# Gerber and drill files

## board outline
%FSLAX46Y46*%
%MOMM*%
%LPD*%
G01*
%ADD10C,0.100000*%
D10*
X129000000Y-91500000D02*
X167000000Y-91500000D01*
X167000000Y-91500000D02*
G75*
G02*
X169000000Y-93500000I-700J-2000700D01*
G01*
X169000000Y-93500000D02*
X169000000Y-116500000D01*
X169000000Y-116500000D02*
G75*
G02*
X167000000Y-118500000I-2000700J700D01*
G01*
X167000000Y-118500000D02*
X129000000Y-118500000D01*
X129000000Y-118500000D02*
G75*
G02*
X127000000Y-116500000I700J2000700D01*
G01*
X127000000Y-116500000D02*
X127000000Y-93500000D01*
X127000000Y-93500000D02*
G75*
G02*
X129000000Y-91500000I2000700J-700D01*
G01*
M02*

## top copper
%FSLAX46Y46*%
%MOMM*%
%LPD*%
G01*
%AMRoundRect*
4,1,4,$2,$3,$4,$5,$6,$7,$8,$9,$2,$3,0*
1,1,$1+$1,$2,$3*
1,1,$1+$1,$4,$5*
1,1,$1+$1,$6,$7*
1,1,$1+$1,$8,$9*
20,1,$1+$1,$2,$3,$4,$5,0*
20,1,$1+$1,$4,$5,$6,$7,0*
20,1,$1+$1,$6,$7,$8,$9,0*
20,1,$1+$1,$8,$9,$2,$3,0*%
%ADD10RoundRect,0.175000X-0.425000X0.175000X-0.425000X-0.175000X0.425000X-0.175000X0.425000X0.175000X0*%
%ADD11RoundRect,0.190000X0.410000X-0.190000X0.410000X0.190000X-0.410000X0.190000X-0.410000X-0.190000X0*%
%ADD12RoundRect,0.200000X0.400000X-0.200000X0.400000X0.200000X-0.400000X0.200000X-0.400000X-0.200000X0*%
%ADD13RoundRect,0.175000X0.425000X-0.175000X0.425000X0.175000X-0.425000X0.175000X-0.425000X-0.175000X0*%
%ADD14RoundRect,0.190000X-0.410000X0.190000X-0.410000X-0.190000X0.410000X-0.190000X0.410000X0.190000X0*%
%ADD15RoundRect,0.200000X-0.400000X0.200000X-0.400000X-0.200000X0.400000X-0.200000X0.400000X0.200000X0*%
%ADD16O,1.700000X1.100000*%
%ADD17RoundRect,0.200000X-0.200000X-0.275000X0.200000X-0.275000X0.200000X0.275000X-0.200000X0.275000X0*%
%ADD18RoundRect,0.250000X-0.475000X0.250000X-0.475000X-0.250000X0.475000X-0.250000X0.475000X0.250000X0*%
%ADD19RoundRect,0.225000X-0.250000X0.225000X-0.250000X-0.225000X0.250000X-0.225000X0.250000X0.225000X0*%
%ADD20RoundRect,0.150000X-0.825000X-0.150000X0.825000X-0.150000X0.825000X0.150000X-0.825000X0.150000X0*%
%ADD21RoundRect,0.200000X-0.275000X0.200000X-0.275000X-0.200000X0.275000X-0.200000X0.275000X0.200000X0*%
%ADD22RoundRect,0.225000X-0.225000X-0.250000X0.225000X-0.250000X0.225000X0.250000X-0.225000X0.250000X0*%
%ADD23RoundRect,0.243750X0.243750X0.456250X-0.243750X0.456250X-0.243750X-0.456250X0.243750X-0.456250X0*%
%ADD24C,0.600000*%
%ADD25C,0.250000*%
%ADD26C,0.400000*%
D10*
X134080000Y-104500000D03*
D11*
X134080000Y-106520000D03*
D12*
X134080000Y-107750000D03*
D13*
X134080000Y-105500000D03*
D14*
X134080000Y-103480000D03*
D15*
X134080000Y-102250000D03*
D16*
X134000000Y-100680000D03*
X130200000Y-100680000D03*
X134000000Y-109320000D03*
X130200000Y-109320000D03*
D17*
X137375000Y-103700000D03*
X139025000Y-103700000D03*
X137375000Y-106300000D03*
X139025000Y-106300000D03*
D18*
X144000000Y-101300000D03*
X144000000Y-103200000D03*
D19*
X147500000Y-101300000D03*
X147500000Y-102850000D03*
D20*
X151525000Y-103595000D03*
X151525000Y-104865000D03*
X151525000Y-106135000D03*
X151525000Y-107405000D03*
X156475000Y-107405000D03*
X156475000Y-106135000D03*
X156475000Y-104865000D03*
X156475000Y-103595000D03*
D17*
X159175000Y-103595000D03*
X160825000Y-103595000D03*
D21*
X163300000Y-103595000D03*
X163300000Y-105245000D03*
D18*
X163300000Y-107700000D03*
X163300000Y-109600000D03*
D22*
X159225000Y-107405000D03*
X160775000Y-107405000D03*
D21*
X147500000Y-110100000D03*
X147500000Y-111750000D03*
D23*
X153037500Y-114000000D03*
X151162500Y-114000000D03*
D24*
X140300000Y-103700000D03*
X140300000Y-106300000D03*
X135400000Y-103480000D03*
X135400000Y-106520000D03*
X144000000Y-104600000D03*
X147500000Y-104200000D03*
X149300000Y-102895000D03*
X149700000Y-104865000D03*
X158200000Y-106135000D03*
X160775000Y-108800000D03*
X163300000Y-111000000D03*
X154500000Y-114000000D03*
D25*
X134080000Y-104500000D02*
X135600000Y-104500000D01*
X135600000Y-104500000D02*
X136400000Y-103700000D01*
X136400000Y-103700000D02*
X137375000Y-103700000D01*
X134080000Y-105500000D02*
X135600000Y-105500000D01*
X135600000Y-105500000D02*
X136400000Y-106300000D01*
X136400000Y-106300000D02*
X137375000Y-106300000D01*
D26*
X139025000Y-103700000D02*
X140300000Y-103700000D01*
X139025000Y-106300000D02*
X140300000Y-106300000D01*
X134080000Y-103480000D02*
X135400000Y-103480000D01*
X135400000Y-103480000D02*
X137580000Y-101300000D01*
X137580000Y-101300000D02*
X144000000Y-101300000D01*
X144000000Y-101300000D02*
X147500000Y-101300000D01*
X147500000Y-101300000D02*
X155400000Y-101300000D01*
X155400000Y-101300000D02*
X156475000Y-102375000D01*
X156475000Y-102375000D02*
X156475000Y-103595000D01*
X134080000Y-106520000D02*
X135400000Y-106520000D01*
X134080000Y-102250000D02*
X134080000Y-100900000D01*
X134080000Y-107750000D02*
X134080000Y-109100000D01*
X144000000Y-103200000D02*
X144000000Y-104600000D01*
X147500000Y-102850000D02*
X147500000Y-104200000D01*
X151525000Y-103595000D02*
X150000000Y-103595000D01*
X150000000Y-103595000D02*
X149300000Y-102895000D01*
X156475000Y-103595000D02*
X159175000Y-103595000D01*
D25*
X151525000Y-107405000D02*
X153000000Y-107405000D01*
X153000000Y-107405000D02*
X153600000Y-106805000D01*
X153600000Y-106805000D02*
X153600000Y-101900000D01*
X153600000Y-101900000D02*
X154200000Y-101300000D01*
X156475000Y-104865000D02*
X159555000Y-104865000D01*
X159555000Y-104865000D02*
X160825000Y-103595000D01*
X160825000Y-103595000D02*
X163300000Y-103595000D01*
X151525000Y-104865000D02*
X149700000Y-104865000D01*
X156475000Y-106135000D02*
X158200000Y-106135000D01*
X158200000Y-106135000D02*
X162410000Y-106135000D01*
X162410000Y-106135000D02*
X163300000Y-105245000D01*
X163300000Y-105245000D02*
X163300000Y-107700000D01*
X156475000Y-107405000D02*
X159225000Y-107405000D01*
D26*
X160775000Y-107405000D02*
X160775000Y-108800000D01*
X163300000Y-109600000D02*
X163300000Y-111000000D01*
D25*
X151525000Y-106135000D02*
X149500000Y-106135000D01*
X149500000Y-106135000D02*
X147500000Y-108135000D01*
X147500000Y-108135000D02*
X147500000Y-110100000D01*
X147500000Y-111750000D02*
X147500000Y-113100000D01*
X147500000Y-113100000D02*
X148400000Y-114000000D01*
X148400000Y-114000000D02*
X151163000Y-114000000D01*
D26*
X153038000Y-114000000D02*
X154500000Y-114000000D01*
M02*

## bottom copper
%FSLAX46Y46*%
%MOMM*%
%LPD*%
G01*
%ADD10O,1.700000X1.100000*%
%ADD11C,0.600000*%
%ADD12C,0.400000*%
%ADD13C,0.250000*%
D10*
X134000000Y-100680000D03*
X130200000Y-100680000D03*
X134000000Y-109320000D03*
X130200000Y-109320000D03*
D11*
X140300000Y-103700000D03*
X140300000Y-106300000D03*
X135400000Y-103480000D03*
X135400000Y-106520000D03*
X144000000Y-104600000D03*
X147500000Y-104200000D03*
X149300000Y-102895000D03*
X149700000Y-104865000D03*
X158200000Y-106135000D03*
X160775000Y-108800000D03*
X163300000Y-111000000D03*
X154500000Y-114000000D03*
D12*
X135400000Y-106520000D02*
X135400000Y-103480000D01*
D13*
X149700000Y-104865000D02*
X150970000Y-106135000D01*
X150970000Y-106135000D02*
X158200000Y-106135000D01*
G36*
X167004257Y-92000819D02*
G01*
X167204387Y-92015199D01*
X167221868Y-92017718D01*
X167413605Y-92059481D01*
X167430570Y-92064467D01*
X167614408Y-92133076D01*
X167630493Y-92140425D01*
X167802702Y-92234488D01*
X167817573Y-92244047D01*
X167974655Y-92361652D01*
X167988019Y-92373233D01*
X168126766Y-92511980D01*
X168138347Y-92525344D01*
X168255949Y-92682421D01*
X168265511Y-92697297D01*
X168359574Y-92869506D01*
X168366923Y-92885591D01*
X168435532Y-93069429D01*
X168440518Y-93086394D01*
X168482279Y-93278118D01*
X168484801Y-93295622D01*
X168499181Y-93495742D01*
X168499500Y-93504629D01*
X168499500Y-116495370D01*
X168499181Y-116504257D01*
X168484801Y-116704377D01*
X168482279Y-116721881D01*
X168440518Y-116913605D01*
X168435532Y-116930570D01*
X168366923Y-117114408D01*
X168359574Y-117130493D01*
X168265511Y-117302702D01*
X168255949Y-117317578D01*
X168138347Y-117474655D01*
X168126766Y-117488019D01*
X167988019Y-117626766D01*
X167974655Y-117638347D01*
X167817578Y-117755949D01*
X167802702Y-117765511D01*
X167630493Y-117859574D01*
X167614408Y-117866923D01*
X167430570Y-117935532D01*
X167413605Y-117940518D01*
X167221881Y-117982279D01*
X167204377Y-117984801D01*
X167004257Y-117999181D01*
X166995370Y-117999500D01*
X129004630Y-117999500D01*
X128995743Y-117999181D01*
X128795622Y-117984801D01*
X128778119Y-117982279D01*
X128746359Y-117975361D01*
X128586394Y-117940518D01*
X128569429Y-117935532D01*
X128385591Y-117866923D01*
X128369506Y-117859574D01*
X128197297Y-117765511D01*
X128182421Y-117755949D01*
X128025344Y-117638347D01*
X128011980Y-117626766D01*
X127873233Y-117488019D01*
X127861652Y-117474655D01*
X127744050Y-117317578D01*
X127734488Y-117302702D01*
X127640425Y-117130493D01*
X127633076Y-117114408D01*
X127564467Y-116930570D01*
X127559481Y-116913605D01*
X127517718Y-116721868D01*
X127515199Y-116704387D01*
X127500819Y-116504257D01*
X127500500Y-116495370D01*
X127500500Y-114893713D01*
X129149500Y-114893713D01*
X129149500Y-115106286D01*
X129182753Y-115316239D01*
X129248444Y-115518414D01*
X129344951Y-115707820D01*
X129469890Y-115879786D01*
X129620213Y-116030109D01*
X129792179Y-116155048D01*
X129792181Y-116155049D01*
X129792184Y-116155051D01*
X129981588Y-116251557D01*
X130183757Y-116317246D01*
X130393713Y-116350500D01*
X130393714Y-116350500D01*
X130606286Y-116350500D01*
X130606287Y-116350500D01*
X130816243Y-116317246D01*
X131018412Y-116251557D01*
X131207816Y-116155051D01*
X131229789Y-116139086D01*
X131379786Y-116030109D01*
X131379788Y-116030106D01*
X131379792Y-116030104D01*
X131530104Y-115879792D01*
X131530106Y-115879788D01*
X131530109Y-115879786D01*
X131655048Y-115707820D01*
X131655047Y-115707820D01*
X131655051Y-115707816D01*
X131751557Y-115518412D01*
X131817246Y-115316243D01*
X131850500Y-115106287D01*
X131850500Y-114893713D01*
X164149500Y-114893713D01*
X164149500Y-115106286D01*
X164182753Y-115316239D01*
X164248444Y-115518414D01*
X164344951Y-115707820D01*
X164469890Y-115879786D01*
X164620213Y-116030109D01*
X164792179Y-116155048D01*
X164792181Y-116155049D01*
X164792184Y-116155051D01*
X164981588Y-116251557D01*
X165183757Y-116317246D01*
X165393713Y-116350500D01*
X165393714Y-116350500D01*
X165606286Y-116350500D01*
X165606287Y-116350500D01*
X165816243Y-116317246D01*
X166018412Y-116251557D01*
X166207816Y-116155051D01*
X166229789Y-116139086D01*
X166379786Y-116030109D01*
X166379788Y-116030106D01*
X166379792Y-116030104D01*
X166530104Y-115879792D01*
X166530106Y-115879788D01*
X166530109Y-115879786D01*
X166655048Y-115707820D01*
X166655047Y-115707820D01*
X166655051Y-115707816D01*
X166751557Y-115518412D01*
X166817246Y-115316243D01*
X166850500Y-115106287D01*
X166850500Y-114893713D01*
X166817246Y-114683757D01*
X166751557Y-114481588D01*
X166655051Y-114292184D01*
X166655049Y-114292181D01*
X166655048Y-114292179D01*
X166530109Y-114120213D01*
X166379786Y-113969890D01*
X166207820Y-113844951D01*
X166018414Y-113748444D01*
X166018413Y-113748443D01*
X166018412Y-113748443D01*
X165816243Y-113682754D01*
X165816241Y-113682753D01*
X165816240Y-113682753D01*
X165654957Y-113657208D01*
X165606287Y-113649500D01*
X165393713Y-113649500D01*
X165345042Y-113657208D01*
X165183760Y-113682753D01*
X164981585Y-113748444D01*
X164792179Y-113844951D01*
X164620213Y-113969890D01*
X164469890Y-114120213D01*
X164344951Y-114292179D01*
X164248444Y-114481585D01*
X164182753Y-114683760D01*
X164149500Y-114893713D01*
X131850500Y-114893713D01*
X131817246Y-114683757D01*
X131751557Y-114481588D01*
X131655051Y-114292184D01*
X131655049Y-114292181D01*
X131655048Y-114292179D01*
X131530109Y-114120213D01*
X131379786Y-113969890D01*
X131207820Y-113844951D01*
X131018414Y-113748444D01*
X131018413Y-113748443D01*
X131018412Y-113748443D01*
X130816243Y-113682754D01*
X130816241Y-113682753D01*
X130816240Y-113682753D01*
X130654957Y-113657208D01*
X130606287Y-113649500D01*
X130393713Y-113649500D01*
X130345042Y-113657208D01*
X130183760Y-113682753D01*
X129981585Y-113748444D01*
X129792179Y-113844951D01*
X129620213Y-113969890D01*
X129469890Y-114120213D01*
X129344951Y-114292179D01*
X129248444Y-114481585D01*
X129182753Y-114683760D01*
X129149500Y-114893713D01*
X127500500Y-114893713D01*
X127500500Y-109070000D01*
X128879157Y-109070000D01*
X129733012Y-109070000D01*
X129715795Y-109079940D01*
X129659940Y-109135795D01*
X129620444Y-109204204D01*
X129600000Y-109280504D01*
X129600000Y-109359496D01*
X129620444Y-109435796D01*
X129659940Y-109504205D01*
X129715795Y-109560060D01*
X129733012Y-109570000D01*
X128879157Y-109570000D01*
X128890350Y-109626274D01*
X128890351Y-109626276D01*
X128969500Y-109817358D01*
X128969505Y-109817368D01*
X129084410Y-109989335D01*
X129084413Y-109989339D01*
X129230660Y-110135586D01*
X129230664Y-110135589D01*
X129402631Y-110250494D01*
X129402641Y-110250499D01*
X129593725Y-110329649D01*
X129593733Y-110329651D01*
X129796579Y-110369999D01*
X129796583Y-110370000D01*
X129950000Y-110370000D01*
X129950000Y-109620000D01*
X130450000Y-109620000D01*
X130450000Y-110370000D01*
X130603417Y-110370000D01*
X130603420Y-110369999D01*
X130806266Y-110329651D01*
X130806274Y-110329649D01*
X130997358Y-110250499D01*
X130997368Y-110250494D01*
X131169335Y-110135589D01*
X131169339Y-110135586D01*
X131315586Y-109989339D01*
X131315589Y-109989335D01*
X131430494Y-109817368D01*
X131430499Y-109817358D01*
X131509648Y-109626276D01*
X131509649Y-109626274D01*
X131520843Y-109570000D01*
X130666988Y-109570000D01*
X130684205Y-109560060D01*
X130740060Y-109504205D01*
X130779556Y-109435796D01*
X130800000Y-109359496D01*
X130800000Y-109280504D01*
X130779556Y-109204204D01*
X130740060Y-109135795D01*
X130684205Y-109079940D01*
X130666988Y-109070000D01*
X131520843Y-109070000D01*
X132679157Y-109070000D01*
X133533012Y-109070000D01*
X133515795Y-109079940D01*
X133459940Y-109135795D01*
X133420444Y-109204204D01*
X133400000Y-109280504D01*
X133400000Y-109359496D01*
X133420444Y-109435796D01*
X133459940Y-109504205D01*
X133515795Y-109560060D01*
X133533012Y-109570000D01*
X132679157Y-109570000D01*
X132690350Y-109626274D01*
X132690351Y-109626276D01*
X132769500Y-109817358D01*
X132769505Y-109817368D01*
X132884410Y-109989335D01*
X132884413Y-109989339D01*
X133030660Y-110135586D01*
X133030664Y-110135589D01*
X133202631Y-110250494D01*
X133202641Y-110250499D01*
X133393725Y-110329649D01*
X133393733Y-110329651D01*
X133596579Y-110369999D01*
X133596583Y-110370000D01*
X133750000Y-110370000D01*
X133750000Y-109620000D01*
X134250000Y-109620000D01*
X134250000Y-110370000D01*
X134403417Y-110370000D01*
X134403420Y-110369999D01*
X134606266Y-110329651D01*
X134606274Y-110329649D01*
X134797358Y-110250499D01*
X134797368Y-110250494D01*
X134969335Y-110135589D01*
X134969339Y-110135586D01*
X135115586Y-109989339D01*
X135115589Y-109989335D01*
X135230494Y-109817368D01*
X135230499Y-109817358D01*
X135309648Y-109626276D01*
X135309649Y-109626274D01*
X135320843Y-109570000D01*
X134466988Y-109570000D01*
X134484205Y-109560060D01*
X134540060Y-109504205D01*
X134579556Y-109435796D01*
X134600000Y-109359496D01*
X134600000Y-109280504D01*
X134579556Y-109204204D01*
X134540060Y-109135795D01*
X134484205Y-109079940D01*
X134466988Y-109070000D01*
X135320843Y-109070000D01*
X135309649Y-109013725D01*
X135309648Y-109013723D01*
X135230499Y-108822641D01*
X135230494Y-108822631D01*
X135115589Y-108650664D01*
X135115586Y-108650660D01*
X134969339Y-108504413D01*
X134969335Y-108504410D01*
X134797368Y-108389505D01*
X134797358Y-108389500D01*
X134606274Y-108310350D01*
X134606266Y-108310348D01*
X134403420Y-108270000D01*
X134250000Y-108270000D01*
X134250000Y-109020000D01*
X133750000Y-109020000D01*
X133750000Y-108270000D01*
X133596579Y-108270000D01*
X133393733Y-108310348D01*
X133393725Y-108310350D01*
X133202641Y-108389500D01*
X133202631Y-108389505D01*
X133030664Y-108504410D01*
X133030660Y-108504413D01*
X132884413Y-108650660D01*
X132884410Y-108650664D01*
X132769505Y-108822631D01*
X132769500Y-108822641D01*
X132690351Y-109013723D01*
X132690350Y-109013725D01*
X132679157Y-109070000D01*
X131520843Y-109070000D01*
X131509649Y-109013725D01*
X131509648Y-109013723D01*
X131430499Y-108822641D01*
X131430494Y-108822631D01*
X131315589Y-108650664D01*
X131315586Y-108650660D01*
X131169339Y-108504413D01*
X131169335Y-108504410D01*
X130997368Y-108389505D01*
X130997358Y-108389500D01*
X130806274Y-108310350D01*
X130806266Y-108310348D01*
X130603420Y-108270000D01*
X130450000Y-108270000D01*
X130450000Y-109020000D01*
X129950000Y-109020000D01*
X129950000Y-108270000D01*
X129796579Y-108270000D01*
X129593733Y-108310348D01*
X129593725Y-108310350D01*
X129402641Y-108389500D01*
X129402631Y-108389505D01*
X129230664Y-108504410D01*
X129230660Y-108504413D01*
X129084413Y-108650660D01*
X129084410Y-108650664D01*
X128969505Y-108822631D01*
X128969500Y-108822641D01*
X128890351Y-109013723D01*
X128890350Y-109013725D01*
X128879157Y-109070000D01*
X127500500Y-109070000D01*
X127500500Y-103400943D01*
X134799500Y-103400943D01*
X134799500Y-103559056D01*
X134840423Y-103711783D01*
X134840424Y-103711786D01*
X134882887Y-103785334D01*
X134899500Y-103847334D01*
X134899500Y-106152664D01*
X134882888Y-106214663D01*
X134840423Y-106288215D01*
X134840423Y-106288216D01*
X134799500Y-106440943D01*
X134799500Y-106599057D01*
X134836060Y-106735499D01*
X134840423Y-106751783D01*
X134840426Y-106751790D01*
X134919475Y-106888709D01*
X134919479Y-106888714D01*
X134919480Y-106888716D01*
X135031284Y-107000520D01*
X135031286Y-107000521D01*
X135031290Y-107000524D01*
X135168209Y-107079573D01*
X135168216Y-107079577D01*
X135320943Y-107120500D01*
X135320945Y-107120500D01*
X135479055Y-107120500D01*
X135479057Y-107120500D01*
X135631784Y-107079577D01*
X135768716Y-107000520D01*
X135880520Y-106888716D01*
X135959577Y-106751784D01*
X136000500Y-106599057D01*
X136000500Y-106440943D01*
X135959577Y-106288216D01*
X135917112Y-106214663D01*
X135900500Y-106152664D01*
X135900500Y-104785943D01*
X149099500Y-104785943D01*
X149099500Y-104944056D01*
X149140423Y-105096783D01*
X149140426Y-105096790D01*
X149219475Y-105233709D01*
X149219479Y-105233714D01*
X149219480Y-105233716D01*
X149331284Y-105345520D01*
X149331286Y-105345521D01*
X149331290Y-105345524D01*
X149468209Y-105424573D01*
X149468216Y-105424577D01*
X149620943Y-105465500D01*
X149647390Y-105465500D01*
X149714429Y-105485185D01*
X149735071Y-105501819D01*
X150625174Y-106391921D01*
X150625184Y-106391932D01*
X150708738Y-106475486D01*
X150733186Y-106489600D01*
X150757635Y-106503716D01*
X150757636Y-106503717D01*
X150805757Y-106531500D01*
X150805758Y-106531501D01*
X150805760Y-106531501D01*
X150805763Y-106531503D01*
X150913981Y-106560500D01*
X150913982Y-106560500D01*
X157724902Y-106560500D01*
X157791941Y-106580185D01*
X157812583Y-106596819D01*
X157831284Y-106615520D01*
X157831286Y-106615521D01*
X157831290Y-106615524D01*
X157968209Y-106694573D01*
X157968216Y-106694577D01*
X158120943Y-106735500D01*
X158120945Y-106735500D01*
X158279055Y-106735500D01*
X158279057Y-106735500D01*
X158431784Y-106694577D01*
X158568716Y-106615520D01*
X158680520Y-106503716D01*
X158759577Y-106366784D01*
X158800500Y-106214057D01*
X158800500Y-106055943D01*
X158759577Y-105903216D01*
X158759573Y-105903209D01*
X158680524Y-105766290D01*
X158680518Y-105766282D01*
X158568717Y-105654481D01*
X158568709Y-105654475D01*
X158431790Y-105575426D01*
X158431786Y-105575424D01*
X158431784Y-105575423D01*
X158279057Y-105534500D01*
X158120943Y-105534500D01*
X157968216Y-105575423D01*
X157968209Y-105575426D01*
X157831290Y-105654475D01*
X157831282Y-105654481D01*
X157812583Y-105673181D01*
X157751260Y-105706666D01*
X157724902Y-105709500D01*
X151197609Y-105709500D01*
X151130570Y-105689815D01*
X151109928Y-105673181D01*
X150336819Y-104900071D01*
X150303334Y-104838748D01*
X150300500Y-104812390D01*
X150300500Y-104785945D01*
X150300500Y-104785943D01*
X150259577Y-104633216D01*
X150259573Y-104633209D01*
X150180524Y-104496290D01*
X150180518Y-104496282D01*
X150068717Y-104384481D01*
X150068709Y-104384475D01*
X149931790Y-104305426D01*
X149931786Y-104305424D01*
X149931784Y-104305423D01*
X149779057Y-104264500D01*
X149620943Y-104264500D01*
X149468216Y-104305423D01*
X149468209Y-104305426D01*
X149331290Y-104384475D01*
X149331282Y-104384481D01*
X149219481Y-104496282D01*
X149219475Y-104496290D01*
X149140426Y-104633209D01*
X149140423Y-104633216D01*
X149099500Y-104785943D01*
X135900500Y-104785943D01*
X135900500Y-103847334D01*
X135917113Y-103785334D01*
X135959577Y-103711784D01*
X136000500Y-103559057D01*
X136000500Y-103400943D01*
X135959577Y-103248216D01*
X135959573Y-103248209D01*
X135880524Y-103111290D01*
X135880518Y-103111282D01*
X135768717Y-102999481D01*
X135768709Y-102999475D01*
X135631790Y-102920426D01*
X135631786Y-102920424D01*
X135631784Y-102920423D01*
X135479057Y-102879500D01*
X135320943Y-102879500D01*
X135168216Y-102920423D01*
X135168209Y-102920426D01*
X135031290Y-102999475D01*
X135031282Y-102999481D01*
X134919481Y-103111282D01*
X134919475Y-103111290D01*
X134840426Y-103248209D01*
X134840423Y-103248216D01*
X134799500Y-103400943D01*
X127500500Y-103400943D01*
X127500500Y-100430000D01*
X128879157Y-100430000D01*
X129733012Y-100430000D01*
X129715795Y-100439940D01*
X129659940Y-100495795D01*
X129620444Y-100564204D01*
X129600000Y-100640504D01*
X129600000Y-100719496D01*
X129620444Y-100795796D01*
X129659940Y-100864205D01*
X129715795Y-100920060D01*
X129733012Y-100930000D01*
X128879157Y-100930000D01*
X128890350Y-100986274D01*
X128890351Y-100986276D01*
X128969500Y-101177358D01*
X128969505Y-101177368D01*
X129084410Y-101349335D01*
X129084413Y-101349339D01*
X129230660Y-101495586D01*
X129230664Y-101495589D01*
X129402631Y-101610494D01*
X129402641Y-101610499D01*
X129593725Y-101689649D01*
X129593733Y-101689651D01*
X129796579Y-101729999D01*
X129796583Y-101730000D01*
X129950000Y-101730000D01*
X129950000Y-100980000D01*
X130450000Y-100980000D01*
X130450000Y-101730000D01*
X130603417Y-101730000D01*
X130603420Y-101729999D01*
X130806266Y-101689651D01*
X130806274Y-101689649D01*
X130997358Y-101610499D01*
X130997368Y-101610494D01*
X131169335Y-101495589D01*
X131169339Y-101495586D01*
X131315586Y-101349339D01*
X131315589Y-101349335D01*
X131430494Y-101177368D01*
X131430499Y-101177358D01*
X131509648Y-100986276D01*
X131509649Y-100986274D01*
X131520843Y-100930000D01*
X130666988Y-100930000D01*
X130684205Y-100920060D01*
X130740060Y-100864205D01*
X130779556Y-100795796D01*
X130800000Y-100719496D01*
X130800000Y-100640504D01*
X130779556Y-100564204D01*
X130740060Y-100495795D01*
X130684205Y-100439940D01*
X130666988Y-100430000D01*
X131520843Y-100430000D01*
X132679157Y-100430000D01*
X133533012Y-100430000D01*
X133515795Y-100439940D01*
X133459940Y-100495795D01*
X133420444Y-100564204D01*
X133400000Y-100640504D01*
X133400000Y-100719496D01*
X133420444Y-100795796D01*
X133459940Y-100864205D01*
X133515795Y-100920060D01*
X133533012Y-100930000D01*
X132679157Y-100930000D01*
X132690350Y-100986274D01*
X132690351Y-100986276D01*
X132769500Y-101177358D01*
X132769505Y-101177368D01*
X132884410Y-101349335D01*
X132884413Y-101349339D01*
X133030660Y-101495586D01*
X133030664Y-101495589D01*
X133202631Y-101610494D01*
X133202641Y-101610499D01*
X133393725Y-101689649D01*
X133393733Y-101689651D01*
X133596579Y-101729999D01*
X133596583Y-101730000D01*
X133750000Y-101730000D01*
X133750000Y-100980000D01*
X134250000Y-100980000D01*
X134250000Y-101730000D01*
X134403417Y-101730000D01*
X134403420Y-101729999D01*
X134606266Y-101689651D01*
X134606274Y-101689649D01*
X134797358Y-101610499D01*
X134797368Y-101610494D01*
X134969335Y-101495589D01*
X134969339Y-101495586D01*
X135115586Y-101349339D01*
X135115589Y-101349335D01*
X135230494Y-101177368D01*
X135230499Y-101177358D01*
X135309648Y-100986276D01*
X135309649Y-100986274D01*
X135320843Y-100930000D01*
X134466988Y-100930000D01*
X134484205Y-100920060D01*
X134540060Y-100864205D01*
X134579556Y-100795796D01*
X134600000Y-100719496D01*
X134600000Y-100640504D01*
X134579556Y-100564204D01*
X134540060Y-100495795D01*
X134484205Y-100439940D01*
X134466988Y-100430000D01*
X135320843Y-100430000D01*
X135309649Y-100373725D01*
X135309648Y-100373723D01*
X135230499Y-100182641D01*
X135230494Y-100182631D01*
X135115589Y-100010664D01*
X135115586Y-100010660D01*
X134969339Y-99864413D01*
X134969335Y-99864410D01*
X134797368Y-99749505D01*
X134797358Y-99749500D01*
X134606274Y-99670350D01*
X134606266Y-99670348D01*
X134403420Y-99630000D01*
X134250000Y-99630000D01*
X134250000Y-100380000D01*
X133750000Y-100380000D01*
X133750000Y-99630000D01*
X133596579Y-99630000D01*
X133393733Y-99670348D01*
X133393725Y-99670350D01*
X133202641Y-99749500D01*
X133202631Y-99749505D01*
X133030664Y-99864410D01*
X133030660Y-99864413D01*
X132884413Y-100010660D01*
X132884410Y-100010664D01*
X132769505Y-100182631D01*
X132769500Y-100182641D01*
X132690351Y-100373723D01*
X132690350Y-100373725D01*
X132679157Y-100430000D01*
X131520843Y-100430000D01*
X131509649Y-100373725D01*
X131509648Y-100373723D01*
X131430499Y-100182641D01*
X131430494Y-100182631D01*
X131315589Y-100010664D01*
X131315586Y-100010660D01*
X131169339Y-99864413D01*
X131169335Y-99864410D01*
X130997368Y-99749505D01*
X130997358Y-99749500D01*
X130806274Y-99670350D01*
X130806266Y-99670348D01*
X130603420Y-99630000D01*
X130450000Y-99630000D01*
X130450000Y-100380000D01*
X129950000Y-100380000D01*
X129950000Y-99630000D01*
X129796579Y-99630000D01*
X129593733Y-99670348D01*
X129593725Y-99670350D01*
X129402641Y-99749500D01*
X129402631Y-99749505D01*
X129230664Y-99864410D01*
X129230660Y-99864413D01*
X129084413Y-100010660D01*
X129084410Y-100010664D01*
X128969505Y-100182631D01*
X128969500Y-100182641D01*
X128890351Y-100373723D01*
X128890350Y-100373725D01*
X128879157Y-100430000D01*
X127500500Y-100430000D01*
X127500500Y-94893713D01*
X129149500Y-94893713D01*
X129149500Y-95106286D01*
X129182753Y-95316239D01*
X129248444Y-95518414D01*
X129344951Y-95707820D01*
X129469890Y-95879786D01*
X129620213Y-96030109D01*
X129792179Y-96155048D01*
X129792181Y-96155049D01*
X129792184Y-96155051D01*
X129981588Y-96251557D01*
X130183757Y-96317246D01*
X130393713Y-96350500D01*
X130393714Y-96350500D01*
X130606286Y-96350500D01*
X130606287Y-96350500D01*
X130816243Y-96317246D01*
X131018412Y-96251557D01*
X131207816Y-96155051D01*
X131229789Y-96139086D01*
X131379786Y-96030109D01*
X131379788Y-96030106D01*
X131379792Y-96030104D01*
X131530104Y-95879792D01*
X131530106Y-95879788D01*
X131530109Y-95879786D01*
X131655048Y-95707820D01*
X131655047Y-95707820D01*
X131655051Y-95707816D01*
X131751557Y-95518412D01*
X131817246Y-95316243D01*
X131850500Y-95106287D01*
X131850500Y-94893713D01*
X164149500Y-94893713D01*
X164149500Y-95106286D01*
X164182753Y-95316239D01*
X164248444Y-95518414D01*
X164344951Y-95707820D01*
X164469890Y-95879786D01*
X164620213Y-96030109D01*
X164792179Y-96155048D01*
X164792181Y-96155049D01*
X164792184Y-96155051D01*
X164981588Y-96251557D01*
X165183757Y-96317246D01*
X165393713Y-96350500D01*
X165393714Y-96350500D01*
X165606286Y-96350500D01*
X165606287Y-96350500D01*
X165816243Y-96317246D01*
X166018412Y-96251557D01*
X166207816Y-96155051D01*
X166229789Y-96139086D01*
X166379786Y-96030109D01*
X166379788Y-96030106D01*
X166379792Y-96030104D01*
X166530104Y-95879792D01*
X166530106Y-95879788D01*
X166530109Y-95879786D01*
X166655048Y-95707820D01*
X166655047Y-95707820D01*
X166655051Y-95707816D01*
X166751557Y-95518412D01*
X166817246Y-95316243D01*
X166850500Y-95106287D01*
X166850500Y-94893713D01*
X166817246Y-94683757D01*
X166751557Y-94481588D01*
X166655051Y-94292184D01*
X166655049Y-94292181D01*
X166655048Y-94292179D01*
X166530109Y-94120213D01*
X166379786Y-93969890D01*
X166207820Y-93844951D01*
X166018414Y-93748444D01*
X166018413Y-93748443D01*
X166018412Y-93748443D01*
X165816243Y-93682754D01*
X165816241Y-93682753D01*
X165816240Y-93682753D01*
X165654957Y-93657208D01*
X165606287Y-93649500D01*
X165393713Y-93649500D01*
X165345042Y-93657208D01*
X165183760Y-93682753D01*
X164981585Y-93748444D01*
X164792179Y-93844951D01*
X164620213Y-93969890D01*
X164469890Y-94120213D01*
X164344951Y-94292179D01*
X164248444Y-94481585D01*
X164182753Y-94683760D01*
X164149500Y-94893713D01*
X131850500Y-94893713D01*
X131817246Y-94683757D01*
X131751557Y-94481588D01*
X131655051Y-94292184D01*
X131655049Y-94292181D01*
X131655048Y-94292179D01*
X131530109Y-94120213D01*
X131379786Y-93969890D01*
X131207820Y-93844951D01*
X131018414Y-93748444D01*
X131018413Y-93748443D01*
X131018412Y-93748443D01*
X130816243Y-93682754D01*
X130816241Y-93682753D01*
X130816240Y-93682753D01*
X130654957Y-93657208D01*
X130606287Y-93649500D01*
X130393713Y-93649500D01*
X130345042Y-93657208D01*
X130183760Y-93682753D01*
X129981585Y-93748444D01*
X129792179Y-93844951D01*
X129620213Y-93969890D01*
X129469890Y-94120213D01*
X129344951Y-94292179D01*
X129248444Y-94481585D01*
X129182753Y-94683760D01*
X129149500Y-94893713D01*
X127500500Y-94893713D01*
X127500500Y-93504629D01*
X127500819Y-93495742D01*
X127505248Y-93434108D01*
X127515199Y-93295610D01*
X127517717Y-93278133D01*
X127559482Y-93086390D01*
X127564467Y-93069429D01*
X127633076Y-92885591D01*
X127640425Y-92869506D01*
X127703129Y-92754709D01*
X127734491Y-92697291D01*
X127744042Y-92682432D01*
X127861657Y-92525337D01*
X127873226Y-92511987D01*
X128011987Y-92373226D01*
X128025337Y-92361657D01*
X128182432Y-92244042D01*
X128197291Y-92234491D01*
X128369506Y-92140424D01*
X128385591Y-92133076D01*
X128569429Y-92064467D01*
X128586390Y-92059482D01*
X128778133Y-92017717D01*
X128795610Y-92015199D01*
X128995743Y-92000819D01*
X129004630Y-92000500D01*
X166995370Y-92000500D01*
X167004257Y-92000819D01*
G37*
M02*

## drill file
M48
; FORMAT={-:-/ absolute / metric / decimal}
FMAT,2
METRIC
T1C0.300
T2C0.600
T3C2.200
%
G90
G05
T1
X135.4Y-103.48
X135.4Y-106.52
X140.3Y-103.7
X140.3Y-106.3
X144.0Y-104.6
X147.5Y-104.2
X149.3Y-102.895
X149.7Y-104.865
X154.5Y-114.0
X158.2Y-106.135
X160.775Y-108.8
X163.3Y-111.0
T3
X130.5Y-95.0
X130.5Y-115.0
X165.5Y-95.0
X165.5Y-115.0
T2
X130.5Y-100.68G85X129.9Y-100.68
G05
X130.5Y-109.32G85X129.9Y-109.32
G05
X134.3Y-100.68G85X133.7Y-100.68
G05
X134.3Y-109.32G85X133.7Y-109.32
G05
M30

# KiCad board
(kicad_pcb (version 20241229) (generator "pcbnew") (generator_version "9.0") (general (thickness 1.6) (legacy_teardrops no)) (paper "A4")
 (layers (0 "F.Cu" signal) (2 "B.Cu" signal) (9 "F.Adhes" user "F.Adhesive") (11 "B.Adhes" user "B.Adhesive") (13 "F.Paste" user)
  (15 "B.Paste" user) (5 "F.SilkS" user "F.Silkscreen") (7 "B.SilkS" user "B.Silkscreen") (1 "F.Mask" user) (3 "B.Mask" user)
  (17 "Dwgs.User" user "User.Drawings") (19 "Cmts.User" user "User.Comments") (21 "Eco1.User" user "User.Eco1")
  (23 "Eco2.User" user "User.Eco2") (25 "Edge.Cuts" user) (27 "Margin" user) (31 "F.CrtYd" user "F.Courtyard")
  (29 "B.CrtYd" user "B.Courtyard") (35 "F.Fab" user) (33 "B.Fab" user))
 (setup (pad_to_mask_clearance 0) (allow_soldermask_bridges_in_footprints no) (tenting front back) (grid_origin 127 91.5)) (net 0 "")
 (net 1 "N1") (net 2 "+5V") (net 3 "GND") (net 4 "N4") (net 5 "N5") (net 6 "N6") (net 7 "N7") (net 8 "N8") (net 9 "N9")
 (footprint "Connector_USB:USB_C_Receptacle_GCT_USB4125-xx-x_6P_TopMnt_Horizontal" (layer "F.Cu") (at 131 105 270)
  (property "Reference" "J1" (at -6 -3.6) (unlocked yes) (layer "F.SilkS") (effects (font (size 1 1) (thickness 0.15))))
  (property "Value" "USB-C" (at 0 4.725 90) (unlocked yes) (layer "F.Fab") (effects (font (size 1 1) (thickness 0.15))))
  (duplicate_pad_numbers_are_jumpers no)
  (pad "A5" smd roundrect (at -0.5 -3.08 270) (size 0.7 1.2) (layers "F.Cu" "F.Mask" "F.Paste") (roundrect_rratio 0.25) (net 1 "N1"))
  (pad "A9" smd roundrect (at 1.52 -3.08 90) (size 0.76 1.2) (layers "F.Cu" "F.Mask" "F.Paste") (roundrect_rratio 0.25) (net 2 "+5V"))
  (pad "A12" smd roundrect (at 2.75 -3.08 90) (size 0.8 1.2) (layers "F.Cu" "F.Mask" "F.Paste") (roundrect_rratio 0.25) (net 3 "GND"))
  (pad "B5" smd roundrect (at 0.5 -3.08 90) (size 0.7 1.2) (layers "F.Cu" "F.Mask" "F.Paste") (roundrect_rratio 0.25) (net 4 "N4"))
  (pad "B9" smd roundrect (at -1.52 -3.08 270) (size 0.76 1.2) (layers "F.Cu" "F.Mask" "F.Paste") (roundrect_rratio 0.25) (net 2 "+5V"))
  (pad "B12" smd roundrect (at -2.75 -3.08 270) (size 0.8 1.2) (layers "F.Cu" "F.Mask" "F.Paste") (roundrect_rratio 0.25) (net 3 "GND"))
  (pad "SH" thru_hole oval (at -4.32 -3 270) (size 1.1 1.7) (drill oval 0.6 1.2) (layers "*.Cu" "*.Mask" "F.Paste")
   (remove_unused_layers no) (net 3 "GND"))
  (pad "SH" thru_hole oval (at -4.32 0.8 270) (size 1.1 1.7) (drill oval 0.6 1.2) (layers "*.Cu" "*.Mask" "F.Paste")
   (remove_unused_layers no) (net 3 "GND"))
  (pad "SH" thru_hole oval (at 4.32 -3 270) (size 1.1 1.7) (drill oval 0.6 1.2) (layers "*.Cu" "*.Mask" "F.Paste") (remove_unused_layers no)
   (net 3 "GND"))
  (pad "SH" thru_hole oval (at 4.32 0.8 270) (size 1.1 1.7) (drill oval 0.6 1.2) (layers "*.Cu" "*.Mask" "F.Paste")
   (remove_unused_layers no) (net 3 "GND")))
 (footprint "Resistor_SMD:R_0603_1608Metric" (layer "F.Cu") (at 138.2 103.7)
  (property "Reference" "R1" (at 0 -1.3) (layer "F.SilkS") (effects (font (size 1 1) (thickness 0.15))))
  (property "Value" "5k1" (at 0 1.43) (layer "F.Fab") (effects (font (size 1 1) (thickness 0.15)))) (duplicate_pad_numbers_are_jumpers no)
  (pad "1" smd roundrect (at -0.825 0) (size 0.8 0.95) (layers "F.Cu" "F.Mask" "F.Paste") (roundrect_rratio 0.25) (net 1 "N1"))
  (pad "2" smd roundrect (at 0.825 0) (size 0.8 0.95) (layers "F.Cu" "F.Mask" "F.Paste") (roundrect_rratio 0.25) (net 3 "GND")))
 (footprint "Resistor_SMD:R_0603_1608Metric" (layer "F.Cu") (at 138.2 106.3)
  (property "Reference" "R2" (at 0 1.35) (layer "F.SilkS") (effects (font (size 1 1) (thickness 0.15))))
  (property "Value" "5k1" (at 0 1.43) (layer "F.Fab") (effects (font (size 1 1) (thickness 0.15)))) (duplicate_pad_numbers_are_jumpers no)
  (pad "1" smd roundrect (at -0.825 0) (size 0.8 0.95) (layers "F.Cu" "F.Mask" "F.Paste") (roundrect_rratio 0.25) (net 4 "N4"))
  (pad "2" smd roundrect (at 0.825 0) (size 0.8 0.95) (layers "F.Cu" "F.Mask" "F.Paste") (roundrect_rratio 0.25) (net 3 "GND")))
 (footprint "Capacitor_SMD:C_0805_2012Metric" (layer "F.Cu") (at 144 102.25 270)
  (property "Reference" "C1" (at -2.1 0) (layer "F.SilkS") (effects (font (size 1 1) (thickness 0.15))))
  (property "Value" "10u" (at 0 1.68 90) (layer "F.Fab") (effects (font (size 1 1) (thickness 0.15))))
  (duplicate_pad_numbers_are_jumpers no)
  (pad "1" smd roundrect (at -0.95 0 270) (size 1 1.45) (layers "F.Cu" "F.Mask" "F.Paste") (roundrect_rratio 0.25) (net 2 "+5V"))
  (pad "2" smd roundrect (at 0.95 0 270) (size 1 1.45) (layers "F.Cu" "F.Mask" "F.Paste") (roundrect_rratio 0.25) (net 3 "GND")))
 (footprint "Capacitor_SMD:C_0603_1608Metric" (layer "F.Cu") (at 147.5 102.075 270)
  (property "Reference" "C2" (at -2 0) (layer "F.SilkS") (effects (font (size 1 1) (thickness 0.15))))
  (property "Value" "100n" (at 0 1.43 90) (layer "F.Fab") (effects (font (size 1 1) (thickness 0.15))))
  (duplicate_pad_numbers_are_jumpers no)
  (pad "1" smd roundrect (at -0.775 0 270) (size 0.9 0.95) (layers "F.Cu" "F.Mask" "F.Paste") (roundrect_rratio 0.25) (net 2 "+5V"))
  (pad "2" smd roundrect (at 0.775 0 270) (size 0.9 0.95) (layers "F.Cu" "F.Mask" "F.Paste") (roundrect_rratio 0.25) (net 3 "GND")))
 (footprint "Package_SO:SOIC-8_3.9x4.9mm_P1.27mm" (layer "F.Cu") (at 154 105.5)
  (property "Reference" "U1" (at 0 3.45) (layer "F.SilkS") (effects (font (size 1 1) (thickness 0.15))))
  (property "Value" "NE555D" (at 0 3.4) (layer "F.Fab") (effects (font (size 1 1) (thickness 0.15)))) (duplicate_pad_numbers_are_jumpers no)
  (pad "1" smd roundrect (at -2.475 -1.905) (size 1.95 0.6) (layers "F.Cu" "F.Mask" "F.Paste") (roundrect_rratio 0.25) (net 3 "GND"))
  (pad "2" smd roundrect (at -2.475 -0.635) (size 1.95 0.6) (layers "F.Cu" "F.Mask" "F.Paste") (roundrect_rratio 0.25) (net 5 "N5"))
  (pad "3" smd roundrect (at -2.475 0.635) (size 1.95 0.6) (layers "F.Cu" "F.Mask" "F.Paste") (roundrect_rratio 0.25) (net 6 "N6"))
  (pad "4" smd roundrect (at -2.475 1.905) (size 1.95 0.6) (layers "F.Cu" "F.Mask" "F.Paste") (roundrect_rratio 0.25) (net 2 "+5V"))
  (pad "5" smd roundrect (at 2.475 1.905) (size 1.95 0.6) (layers "F.Cu" "F.Mask" "F.Paste") (roundrect_rratio 0.25) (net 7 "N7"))
  (pad "6" smd roundrect (at 2.475 0.635) (size 1.95 0.6) (layers "F.Cu" "F.Mask" "F.Paste") (roundrect_rratio 0.25) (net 5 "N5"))
  (pad "7" smd roundrect (at 2.475 -0.635) (size 1.95 0.6) (layers "F.Cu" "F.Mask" "F.Paste") (roundrect_rratio 0.25) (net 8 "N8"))
  (pad "8" smd roundrect (at 2.475 -1.905) (size 1.95 0.6) (layers "F.Cu" "F.Mask" "F.Paste") (roundrect_rratio 0.25) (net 2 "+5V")))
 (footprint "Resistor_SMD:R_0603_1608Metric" (layer "F.Cu") (at 160 103.595)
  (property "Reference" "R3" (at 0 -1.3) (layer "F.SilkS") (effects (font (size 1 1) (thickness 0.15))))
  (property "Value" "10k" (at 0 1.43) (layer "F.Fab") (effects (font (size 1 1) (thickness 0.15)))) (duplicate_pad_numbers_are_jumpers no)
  (pad "1" smd roundrect (at -0.825 0) (size 0.8 0.95) (layers "F.Cu" "F.Mask" "F.Paste") (roundrect_rratio 0.25) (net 2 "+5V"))
  (pad "2" smd roundrect (at 0.825 0) (size 0.8 0.95) (layers "F.Cu" "F.Mask" "F.Paste") (roundrect_rratio 0.25) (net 8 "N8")))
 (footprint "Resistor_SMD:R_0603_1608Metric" (layer "F.Cu") (at 163.3 104.42 270)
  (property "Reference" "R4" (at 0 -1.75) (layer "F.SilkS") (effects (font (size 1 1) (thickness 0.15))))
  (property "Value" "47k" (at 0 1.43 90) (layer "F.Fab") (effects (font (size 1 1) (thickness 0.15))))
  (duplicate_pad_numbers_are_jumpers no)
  (pad "1" smd roundrect (at -0.825 0 270) (size 0.8 0.95) (layers "F.Cu" "F.Mask" "F.Paste") (roundrect_rratio 0.25) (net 8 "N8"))
  (pad "2" smd roundrect (at 0.825 0 270) (size 0.8 0.95) (layers "F.Cu" "F.Mask" "F.Paste") (roundrect_rratio 0.25) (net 5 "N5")))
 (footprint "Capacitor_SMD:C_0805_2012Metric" (layer "F.Cu") (at 163.3 108.65 270)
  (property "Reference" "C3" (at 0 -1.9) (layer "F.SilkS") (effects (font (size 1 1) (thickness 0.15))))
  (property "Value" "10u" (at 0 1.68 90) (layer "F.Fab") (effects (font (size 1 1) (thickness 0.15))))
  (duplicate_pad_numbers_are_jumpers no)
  (pad "1" smd roundrect (at -0.95 0 270) (size 1 1.45) (layers "F.Cu" "F.Mask" "F.Paste") (roundrect_rratio 0.25) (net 5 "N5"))
  (pad "2" smd roundrect (at 0.95 0 270) (size 1 1.45) (layers "F.Cu" "F.Mask" "F.Paste") (roundrect_rratio 0.25) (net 3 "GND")))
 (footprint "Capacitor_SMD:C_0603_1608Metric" (layer "F.Cu") (at 160 107.405)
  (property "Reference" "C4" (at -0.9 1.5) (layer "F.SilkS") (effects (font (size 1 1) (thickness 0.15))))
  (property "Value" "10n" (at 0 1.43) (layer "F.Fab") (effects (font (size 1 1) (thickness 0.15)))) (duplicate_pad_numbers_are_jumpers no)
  (pad "1" smd roundrect (at -0.775 0) (size 0.9 0.95) (layers "F.Cu" "F.Mask" "F.Paste") (roundrect_rratio 0.25) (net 7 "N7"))
  (pad "2" smd roundrect (at 0.775 0) (size 0.9 0.95) (layers "F.Cu" "F.Mask" "F.Paste") (roundrect_rratio 0.25) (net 3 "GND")))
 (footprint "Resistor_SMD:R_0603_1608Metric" (layer "F.Cu") (at 147.5 110.925 270)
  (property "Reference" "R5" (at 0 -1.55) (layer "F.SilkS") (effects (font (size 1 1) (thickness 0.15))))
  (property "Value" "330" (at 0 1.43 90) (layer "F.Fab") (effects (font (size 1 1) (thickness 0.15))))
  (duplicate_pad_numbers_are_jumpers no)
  (pad "1" smd roundrect (at -0.825 0 270) (size 0.8 0.95) (layers "F.Cu" "F.Mask" "F.Paste") (roundrect_rratio 0.25) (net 6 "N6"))
  (pad "2" smd roundrect (at 0.825 0 270) (size 0.8 0.95) (layers "F.Cu" "F.Mask" "F.Paste") (roundrect_rratio 0.25) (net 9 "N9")))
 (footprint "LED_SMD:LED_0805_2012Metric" (layer "F.Cu") (at 152.1 114 180)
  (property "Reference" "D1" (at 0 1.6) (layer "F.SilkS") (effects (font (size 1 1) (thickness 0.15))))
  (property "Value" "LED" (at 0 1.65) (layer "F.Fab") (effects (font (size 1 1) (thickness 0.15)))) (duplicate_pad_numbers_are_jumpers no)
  (pad "1" smd roundrect (at -0.9375 0 180) (size 0.975 1.4) (layers "F.Cu" "F.Mask" "F.Paste") (roundrect_rratio 0.25) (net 3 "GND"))
  (pad "2" smd roundrect (at 0.9375 0 180) (size 0.975 1.4) (layers "F.Cu" "F.Mask" "F.Paste") (roundrect_rratio 0.25) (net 9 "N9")))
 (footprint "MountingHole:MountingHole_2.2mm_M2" (layer "F.Cu") (at 130.5 95)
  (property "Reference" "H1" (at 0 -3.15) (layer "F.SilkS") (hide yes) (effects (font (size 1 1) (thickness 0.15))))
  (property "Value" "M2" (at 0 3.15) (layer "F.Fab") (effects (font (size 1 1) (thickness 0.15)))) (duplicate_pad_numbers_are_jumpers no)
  (pad "" np_thru_hole circle (at 0 0) (size 2.2 2.2) (drill 2.2) (layers "*.Cu" "*.Mask")))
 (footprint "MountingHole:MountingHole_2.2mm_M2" (layer "F.Cu") (at 165.5 95)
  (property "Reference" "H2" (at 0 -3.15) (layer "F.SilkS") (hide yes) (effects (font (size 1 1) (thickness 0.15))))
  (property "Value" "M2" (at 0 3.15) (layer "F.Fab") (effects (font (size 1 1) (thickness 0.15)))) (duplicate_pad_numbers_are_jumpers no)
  (pad "" np_thru_hole circle (at 0 0) (size 2.2 2.2) (drill 2.2) (layers "*.Cu" "*.Mask")))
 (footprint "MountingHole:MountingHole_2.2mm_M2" (layer "F.Cu") (at 130.5 115)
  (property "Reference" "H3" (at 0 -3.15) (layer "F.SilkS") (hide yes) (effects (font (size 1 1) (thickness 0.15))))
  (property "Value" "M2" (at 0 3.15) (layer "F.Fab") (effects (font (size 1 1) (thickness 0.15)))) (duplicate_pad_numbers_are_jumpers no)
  (pad "" np_thru_hole circle (at 0 0) (size 2.2 2.2) (drill 2.2) (layers "*.Cu" "*.Mask")))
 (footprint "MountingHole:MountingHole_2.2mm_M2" (layer "F.Cu") (at 165.5 115)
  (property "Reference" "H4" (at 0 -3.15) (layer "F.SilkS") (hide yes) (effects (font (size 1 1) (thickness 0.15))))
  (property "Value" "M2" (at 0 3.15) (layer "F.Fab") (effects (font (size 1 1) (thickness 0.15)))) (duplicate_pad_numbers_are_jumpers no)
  (pad "" np_thru_hole circle (at 0 0) (size 2.2 2.2) (drill 2.2) (layers "*.Cu" "*.Mask")))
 (segment (start 134.08 104.5) (end 135.6 104.5) (width 0.25) (layer "F.Cu") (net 1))
 (segment (start 135.6 104.5) (end 136.4 103.7) (width 0.25) (layer "F.Cu") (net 1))
 (segment (start 136.4 103.7) (end 137.375 103.7) (width 0.25) (layer "F.Cu") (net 1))
 (segment (start 134.08 105.5) (end 135.6 105.5) (width 0.25) (layer "F.Cu") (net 4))
 (segment (start 135.6 105.5) (end 136.4 106.3) (width 0.25) (layer "F.Cu") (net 4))
 (segment (start 136.4 106.3) (end 137.375 106.3) (width 0.25) (layer "F.Cu") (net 4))
 (segment (start 139.025 103.7) (end 140.3 103.7) (width 0.4) (layer "F.Cu") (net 3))
 (via (at 140.3 103.7) (size 0.6) (drill 0.3) (layers "F.Cu" "B.Cu") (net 3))
 (segment (start 139.025 106.3) (end 140.3 106.3) (width 0.4) (layer "F.Cu") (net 3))
 (via (at 140.3 106.3) (size 0.6) (drill 0.3) (layers "F.Cu" "B.Cu") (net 3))
 (segment (start 134.08 103.48) (end 135.4 103.48) (width 0.4) (layer "F.Cu") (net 2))
 (via (at 135.4 103.48) (size 0.6) (drill 0.3) (layers "F.Cu" "B.Cu") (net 2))
 (segment (start 135.4 103.48) (end 137.58 101.3) (width 0.4) (layer "F.Cu") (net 2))
 (segment (start 137.58 101.3) (end 144 101.3) (width 0.4) (layer "F.Cu") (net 2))
 (segment (start 144 101.3) (end 147.5 101.3) (width 0.4) (layer "F.Cu") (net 2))
 (segment (start 147.5 101.3) (end 155.4 101.3) (width 0.4) (layer "F.Cu") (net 2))
 (segment (start 155.4 101.3) (end 156.475 102.375) (width 0.4) (layer "F.Cu") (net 2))
 (segment (start 156.475 102.375) (end 156.475 103.595) (width 0.4) (layer "F.Cu") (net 2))
 (segment (start 134.08 106.52) (end 135.4 106.52) (width 0.4) (layer "F.Cu") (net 2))
 (via (at 135.4 106.52) (size 0.6) (drill 0.3) (layers "F.Cu" "B.Cu") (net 2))
 (segment (start 135.4 106.52) (end 135.4 103.48) (width 0.4) (layer "B.Cu") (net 2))
 (segment (start 134.08 102.25) (end 134.08 100.9) (width 0.4) (layer "F.Cu") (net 3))
 (segment (start 134.08 107.75) (end 134.08 109.1) (width 0.4) (layer "F.Cu") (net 3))
 (segment (start 144 103.2) (end 144 104.6) (width 0.4) (layer "F.Cu") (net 3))
 (via (at 144 104.6) (size 0.6) (drill 0.3) (layers "F.Cu" "B.Cu") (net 3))
 (segment (start 147.5 102.85) (end 147.5 104.2) (width 0.4) (layer "F.Cu") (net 3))
 (via (at 147.5 104.2) (size 0.6) (drill 0.3) (layers "F.Cu" "B.Cu") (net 3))
 (segment (start 151.525 103.595) (end 150 103.595) (width 0.4) (layer "F.Cu") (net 3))
 (segment (start 150 103.595) (end 149.3 102.895) (width 0.4) (layer "F.Cu") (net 3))
 (via (at 149.3 102.895) (size 0.6) (drill 0.3) (layers "F.Cu" "B.Cu") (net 3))
 (segment (start 156.475 103.595) (end 159.175 103.595) (width 0.4) (layer "F.Cu") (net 2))
 (segment (start 151.525 107.405) (end 153 107.405) (width 0.25) (layer "F.Cu") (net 2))
 (segment (start 153 107.405) (end 153.6 106.805) (width 0.25) (layer "F.Cu") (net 2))
 (segment (start 153.6 106.805) (end 153.6 101.9) (width 0.25) (layer "F.Cu") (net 2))
 (segment (start 153.6 101.9) (end 154.2 101.3) (width 0.25) (layer "F.Cu") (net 2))
 (segment (start 156.475 104.865) (end 159.555 104.865) (width 0.25) (layer "F.Cu") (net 8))
 (segment (start 159.555 104.865) (end 160.825 103.595) (width 0.25) (layer "F.Cu") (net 8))
 (segment (start 160.825 103.595) (end 163.3 103.595) (width 0.25) (layer "F.Cu") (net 8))
 (segment (start 151.525 104.865) (end 149.7 104.865) (width 0.25) (layer "F.Cu") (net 5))
 (via (at 149.7 104.865) (size 0.6) (drill 0.3) (layers "F.Cu" "B.Cu") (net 5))
 (segment (start 149.7 104.865) (end 150.97 106.135) (width 0.25) (layer "B.Cu") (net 5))
 (segment (start 150.97 106.135) (end 158.2 106.135) (width 0.25) (layer "B.Cu") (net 5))
 (via (at 158.2 106.135) (size 0.6) (drill 0.3) (layers "F.Cu" "B.Cu") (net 5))
 (segment (start 156.475 106.135) (end 158.2 106.135) (width 0.25) (layer "F.Cu") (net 5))
 (segment (start 158.2 106.135) (end 162.41 106.135) (width 0.25) (layer "F.Cu") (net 5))
 (segment (start 162.41 106.135) (end 163.3 105.245) (width 0.25) (layer "F.Cu") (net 5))
 (segment (start 163.3 105.245) (end 163.3 107.7) (width 0.25) (layer "F.Cu") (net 5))
 (segment (start 156.475 107.405) (end 159.225 107.405) (width 0.25) (layer "F.Cu") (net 7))
 (segment (start 160.775 107.405) (end 160.775 108.8) (width 0.4) (layer "F.Cu") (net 3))
 (via (at 160.775 108.8) (size 0.6) (drill 0.3) (layers "F.Cu" "B.Cu") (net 3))
 (segment (start 163.3 109.6) (end 163.3 111) (width 0.4) (layer "F.Cu") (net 3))
 (via (at 163.3 111) (size 0.6) (drill 0.3) (layers "F.Cu" "B.Cu") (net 3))
 (segment (start 151.525 106.135) (end 149.5 106.135) (width 0.25) (layer "F.Cu") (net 6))
 (segment (start 149.5 106.135) (end 147.5 108.135) (width 0.25) (layer "F.Cu") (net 6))
 (segment (start 147.5 108.135) (end 147.5 110.1) (width 0.25) (layer "F.Cu") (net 6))
 (segment (start 147.5 111.75) (end 147.5 113.1) (width 0.25) (layer "F.Cu") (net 9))
 (segment (start 147.5 113.1) (end 148.4 114) (width 0.25) (layer "F.Cu") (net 9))
 (segment (start 148.4 114) (end 151.163 114) (width 0.25) (layer "F.Cu") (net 9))
 (segment (start 153.038 114) (end 154.5 114) (width 0.4) (layer "F.Cu") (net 3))
 (via (at 154.5 114) (size 0.6) (drill 0.3) (layers "F.Cu" "B.Cu") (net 3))
 (gr_line (start 129 91.5) (end 167 91.5) (stroke (width 0.1) (type default)) (layer "Edge.Cuts"))
 (gr_arc (start 167 91.5) (mid 168.414 92.086) (end 169 93.5) (stroke (width 0.1) (type default)) (layer "Edge.Cuts"))
 (gr_line (start 169 93.5) (end 169 116.5) (stroke (width 0.1) (type default)) (layer "Edge.Cuts"))
 (gr_arc (start 169 116.5) (mid 168.414 117.914) (end 167 118.5) (stroke (width 0.1) (type default)) (layer "Edge.Cuts"))
 (gr_line (start 167 118.5) (end 129 118.5) (stroke (width 0.1) (type default)) (layer "Edge.Cuts"))
 (gr_arc (start 129 118.5) (mid 127.586 117.914) (end 127 116.5) (stroke (width 0.1) (type default)) (layer "Edge.Cuts"))
 (gr_line (start 127 116.5) (end 127 93.5) (stroke (width 0.1) (type default)) (layer "Edge.Cuts"))
 (gr_arc (start 127 93.5) (mid 127.586 92.086) (end 129 91.5) (stroke (width 0.1) (type default)) (layer "Edge.Cuts"))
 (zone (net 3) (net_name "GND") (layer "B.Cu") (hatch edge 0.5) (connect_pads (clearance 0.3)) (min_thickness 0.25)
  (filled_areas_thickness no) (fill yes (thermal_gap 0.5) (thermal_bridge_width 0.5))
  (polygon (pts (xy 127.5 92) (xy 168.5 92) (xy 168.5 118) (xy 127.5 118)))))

